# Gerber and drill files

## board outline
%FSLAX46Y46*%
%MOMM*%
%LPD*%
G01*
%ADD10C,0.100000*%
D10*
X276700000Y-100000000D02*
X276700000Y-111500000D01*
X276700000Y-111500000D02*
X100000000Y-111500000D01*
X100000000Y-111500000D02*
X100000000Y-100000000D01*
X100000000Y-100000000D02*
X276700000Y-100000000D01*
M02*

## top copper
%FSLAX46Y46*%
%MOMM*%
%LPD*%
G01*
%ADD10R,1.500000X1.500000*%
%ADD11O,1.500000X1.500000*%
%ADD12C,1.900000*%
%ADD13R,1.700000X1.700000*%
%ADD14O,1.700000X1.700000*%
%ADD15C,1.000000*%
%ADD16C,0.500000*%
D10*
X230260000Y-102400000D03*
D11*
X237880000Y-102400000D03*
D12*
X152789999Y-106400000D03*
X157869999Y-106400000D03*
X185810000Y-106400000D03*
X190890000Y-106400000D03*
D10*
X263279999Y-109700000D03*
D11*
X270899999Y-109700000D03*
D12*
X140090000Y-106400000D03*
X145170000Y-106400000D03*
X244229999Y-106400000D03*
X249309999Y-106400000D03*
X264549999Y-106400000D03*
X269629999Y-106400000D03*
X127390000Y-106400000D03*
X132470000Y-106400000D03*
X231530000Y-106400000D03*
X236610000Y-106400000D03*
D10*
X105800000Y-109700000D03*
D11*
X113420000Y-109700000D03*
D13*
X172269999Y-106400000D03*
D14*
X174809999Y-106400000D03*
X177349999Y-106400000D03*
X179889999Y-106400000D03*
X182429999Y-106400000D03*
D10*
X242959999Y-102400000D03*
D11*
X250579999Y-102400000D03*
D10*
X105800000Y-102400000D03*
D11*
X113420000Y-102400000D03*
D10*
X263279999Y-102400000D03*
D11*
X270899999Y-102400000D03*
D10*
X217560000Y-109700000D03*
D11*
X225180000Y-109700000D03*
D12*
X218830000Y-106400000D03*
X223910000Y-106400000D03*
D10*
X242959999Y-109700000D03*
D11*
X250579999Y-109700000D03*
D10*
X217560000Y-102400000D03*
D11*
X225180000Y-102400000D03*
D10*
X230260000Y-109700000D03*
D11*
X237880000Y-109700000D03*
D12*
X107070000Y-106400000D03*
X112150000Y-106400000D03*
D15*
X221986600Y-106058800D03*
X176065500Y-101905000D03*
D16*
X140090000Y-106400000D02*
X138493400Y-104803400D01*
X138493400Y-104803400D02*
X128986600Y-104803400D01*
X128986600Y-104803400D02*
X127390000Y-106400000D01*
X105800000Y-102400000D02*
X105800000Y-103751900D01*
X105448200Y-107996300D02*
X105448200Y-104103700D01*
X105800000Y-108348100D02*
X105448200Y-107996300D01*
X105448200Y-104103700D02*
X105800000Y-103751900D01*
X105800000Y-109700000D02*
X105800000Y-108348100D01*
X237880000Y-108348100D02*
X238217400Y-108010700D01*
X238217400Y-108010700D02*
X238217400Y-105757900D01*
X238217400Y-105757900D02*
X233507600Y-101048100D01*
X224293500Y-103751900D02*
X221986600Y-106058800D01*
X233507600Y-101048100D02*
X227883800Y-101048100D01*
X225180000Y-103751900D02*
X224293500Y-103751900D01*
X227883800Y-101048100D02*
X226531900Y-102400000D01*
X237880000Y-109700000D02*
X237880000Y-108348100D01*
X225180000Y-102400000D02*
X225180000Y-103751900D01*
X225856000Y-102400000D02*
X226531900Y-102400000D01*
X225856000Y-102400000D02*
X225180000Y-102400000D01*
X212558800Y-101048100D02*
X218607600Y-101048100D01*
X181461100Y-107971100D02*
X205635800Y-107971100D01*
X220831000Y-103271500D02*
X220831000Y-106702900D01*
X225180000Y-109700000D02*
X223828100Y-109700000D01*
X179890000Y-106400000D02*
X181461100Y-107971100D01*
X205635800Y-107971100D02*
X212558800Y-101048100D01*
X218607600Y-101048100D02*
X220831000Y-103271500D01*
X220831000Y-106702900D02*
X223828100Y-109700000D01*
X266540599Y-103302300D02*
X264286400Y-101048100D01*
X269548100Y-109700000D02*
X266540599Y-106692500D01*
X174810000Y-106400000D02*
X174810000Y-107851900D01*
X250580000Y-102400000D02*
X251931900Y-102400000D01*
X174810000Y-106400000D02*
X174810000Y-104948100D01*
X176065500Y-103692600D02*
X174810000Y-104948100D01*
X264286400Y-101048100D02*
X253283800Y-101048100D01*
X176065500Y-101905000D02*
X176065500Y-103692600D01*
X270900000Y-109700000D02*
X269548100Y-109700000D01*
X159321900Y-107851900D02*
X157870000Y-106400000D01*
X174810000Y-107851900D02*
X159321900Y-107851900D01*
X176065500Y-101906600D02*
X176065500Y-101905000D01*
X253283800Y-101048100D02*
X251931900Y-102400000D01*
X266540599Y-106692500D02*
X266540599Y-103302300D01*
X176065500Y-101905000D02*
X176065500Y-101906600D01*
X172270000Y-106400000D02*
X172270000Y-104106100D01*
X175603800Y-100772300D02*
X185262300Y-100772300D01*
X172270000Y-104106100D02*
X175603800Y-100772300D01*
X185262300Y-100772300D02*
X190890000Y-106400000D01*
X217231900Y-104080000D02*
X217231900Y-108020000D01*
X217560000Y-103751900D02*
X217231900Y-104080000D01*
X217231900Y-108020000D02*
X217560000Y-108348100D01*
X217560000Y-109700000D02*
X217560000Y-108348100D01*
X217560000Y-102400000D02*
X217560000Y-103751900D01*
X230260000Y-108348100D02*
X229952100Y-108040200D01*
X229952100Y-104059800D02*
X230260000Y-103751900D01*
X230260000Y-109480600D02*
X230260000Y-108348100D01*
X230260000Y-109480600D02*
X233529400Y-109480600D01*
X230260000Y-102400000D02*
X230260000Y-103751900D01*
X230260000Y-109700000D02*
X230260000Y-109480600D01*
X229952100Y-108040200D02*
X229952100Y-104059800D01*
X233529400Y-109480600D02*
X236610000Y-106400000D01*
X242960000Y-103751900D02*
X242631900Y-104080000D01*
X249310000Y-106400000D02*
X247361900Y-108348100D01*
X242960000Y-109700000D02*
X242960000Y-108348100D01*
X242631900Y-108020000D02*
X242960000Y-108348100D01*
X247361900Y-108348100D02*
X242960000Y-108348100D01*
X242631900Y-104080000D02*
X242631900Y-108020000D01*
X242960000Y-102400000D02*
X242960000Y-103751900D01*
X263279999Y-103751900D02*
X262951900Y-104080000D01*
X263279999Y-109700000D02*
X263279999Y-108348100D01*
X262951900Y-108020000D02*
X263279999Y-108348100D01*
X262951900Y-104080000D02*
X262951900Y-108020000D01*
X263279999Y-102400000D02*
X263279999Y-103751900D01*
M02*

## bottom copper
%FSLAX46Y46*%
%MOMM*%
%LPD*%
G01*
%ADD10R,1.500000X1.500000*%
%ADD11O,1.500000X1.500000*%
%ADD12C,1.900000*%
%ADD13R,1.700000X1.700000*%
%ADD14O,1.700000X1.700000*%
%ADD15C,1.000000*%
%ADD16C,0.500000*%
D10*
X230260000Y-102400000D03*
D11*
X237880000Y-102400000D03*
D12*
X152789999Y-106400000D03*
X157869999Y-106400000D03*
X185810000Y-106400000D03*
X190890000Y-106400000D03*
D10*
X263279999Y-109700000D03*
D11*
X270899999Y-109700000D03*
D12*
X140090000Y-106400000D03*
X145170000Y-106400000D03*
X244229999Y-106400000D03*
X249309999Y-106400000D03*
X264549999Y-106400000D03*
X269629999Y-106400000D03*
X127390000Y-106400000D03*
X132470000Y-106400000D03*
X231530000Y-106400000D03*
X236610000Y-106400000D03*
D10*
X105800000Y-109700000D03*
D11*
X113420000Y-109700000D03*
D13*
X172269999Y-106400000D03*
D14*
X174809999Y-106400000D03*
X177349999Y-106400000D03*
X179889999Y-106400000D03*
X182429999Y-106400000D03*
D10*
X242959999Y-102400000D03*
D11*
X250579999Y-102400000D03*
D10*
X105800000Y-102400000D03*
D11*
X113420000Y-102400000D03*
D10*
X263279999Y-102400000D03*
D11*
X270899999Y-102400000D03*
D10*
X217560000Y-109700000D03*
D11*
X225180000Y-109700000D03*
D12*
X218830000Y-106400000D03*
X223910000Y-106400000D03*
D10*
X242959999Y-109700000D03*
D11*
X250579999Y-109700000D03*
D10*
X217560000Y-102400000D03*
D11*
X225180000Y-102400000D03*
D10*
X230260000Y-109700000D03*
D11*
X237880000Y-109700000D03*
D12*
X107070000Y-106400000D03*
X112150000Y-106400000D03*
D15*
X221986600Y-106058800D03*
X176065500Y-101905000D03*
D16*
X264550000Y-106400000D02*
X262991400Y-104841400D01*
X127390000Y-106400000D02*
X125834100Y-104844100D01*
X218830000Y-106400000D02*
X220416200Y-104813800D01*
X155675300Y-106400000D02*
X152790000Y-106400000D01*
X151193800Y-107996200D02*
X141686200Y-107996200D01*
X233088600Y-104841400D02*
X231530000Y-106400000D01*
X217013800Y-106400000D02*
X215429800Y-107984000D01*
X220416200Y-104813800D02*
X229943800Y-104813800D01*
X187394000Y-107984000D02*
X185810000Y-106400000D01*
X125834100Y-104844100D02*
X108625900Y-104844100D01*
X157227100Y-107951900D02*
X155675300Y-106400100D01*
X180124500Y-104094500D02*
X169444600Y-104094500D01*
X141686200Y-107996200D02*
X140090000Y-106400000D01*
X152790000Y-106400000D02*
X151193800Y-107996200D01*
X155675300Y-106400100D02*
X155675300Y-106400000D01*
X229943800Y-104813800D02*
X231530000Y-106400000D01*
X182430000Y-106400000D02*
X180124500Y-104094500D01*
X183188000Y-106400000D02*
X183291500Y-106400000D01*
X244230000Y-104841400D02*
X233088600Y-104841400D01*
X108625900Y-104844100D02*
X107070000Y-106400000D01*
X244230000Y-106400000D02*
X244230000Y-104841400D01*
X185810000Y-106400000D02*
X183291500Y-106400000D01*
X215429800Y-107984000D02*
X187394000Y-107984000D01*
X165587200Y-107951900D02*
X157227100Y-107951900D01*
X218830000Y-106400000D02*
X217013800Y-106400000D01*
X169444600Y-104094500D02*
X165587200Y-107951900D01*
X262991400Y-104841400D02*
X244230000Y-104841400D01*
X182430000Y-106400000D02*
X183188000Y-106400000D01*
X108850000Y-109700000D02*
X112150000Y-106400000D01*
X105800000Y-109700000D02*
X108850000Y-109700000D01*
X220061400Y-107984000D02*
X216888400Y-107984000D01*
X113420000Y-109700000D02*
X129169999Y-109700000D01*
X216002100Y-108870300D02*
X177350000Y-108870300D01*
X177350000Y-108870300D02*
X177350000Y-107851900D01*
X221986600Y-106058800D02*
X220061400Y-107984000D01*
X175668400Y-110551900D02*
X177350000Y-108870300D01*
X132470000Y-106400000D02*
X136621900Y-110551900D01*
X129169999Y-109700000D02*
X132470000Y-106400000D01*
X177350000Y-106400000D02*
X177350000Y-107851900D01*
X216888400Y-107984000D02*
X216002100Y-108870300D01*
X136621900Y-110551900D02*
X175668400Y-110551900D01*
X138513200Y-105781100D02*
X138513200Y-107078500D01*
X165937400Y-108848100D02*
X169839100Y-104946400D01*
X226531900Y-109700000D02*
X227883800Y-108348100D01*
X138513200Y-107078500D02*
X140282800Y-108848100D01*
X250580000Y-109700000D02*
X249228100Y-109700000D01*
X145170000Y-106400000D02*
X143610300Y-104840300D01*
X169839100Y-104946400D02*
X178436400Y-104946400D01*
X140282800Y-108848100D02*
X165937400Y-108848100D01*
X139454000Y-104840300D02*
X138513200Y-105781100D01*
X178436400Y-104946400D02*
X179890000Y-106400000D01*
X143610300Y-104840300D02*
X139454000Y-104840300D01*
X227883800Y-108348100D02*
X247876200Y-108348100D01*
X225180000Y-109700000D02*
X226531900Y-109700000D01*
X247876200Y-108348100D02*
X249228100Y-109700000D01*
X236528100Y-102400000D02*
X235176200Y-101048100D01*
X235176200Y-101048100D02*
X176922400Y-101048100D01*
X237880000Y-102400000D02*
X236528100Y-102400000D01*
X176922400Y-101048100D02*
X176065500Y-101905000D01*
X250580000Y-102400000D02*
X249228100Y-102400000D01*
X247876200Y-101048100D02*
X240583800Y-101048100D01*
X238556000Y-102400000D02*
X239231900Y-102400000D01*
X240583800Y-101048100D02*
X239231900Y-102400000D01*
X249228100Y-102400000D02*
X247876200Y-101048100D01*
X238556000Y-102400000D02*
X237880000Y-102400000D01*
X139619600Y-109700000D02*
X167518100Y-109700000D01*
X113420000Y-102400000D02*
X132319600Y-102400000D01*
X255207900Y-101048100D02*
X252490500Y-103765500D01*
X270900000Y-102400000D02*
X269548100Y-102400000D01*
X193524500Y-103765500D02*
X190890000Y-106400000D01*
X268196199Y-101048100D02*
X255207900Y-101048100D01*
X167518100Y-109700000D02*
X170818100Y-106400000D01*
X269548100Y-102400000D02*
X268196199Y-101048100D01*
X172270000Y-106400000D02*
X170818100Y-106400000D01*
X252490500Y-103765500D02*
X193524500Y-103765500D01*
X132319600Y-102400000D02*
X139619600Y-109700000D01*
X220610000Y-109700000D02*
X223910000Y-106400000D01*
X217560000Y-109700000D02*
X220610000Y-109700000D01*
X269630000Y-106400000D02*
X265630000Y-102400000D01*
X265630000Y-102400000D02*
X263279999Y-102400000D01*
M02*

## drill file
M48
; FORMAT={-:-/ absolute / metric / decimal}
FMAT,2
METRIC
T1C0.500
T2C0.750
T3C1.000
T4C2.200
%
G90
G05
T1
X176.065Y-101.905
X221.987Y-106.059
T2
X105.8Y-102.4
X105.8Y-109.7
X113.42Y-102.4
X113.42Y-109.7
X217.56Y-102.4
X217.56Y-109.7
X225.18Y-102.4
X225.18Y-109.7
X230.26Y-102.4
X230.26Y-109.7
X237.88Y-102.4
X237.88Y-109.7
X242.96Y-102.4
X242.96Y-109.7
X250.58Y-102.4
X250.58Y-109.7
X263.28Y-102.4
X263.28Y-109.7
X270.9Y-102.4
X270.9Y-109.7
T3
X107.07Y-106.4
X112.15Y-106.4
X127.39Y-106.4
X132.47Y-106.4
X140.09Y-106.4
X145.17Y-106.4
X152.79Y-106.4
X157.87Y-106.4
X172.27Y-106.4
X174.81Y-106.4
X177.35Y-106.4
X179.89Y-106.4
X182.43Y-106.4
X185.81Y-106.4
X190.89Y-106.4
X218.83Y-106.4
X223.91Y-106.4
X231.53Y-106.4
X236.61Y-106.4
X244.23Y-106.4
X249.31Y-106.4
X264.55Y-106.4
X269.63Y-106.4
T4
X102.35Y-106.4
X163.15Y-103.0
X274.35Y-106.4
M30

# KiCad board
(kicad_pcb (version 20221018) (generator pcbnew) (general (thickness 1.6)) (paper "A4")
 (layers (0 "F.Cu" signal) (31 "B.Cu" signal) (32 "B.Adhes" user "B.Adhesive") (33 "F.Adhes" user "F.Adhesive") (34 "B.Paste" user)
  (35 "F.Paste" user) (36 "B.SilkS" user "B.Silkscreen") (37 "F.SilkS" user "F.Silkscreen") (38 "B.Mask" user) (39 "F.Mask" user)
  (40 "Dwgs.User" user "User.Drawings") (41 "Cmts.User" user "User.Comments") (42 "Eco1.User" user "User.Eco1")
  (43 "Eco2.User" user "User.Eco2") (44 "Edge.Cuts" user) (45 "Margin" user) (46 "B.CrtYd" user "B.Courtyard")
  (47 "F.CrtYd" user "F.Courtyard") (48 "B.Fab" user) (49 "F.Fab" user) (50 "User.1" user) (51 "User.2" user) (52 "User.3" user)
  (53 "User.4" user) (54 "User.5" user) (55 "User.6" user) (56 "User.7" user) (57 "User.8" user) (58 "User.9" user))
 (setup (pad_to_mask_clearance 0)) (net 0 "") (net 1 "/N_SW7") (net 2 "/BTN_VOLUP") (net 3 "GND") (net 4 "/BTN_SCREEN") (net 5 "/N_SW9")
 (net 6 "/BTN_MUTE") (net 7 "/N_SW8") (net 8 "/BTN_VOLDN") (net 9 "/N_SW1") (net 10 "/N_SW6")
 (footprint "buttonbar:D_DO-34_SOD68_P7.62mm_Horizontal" (layer "F.Cu") (at 230.26 102.4)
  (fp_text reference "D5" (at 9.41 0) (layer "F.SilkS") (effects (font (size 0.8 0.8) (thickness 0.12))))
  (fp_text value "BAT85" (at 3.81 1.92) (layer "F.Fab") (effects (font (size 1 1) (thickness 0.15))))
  (pad "1" thru_hole rect (at 0 0) (size 1.5 1.5) (drill 0.75) (layers "*.Cu" "*.Mask") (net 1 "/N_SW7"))
  (pad "2" thru_hole oval (at 7.62 0) (size 1.5 1.5) (drill 0.75) (layers "*.Cu" "*.Mask") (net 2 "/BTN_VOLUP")))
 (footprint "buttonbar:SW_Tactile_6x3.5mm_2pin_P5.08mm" (layer "F.Cu") (at 155.329999 106.4)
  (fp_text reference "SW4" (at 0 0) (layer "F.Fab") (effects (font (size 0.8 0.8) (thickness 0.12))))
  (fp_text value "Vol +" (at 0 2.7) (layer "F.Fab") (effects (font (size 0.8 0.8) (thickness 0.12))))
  (pad "1" thru_hole circle (at -2.54 0) (size 1.9 1.9) (drill 1) (layers "*.Cu" "*.Mask") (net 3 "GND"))
  (pad "2" thru_hole circle (at 2.54 0) (size 1.9 1.9) (drill 1) (layers "*.Cu" "*.Mask") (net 2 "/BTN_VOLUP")))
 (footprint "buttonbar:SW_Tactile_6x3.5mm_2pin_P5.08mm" (layer "F.Cu") (at 188.35 106.4)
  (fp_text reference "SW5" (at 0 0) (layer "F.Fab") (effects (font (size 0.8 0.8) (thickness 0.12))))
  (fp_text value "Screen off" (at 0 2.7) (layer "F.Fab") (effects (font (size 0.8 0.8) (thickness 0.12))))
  (pad "1" thru_hole circle (at -2.54 0) (size 1.9 1.9) (drill 1) (layers "*.Cu" "*.Mask") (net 3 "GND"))
  (pad "2" thru_hole circle (at 2.54 0) (size 1.9 1.9) (drill 1) (layers "*.Cu" "*.Mask") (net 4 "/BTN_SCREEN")))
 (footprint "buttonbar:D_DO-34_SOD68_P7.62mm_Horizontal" (layer "F.Cu") (at 263.279999 109.7)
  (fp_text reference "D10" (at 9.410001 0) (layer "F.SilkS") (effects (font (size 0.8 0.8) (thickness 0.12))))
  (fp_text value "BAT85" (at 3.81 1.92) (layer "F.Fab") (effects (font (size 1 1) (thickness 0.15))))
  (pad "1" thru_hole rect (at 0 0) (size 1.5 1.5) (drill 0.75) (layers "*.Cu" "*.Mask") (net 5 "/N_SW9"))
  (pad "2" thru_hole oval (at 7.62 0) (size 1.5 1.5) (drill 0.75) (layers "*.Cu" "*.Mask") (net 2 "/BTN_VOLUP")))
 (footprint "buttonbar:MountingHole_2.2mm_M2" (layer "F.Cu") (at 163.15 103)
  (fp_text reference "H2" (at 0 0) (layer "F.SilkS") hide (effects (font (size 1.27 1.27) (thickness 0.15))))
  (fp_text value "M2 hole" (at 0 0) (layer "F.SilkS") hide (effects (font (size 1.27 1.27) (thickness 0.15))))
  (pad "" np_thru_hole circle (at 0 0) (size 2.2 2.2) (drill 2.2) (layers "F&B.Cu" "*.Mask")))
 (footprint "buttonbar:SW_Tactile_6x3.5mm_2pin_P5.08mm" (layer "F.Cu") (at 142.63 106.4)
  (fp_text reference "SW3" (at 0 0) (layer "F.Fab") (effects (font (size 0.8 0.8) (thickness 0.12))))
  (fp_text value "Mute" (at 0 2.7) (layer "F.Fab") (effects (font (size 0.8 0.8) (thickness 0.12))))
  (pad "1" thru_hole circle (at -2.54 0) (size 1.9 1.9) (drill 1) (layers "*.Cu" "*.Mask") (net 3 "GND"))
  (pad "2" thru_hole circle (at 2.54 0) (size 1.9 1.9) (drill 1) (layers "*.Cu" "*.Mask") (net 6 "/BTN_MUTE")))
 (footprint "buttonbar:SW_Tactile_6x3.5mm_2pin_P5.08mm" (layer "F.Cu") (at 246.769999 106.4)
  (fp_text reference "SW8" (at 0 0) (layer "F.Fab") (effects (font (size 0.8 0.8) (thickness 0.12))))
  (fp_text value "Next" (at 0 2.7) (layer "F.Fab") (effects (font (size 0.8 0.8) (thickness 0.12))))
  (pad "1" thru_hole circle (at -2.54 0) (size 1.9 1.9) (drill 1) (layers "*.Cu" "*.Mask") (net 3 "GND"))
  (pad "2" thru_hole circle (at 2.54 0) (size 1.9 1.9) (drill 1) (layers "*.Cu" "*.Mask") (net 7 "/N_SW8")))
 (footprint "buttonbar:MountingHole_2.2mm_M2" (layer "F.Cu") (at 102.35 106.4)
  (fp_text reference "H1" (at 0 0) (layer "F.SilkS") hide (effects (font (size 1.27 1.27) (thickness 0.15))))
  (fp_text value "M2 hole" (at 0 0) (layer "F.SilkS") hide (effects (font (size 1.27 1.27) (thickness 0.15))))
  (pad "" np_thru_hole circle (at 0 0) (size 2.2 2.2) (drill 2.2) (layers "F&B.Cu" "*.Mask")))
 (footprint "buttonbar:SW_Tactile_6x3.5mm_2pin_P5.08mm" (layer "F.Cu") (at 267.089999 106.4)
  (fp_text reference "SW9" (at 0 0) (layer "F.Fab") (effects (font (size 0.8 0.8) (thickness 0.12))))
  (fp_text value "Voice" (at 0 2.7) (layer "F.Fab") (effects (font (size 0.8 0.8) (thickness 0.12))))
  (pad "1" thru_hole circle (at -2.54 0) (size 1.9 1.9) (drill 1) (layers "*.Cu" "*.Mask") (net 3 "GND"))
  (pad "2" thru_hole circle (at 2.54 0) (size 1.9 1.9) (drill 1) (layers "*.Cu" "*.Mask") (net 5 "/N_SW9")))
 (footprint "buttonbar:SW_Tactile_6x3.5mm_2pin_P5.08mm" (layer "F.Cu") (at 129.93 106.4)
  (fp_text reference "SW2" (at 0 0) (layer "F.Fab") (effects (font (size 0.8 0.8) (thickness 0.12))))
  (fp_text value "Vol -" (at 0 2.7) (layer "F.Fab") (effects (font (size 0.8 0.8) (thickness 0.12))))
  (pad "1" thru_hole circle (at -2.54 0) (size 1.9 1.9) (drill 1) (layers "*.Cu" "*.Mask") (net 3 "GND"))
  (pad "2" thru_hole circle (at 2.54 0) (size 1.9 1.9) (drill 1) (layers "*.Cu" "*.Mask") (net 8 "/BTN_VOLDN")))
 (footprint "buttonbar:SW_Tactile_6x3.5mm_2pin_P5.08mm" (layer "F.Cu") (at 234.07 106.4)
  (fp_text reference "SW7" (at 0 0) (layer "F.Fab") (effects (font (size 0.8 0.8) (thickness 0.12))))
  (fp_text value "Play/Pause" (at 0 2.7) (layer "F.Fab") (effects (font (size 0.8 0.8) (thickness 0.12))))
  (pad "1" thru_hole circle (at -2.54 0) (size 1.9 1.9) (drill 1) (layers "*.Cu" "*.Mask") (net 3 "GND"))
  (pad "2" thru_hole circle (at 2.54 0) (size 1.9 1.9) (drill 1) (layers "*.Cu" "*.Mask") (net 1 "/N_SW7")))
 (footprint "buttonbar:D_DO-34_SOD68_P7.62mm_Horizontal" (layer "F.Cu") (at 105.8 109.7)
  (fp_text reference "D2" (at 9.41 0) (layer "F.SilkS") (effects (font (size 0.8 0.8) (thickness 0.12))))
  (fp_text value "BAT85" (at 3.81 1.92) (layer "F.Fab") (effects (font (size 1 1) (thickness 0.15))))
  (pad "1" thru_hole rect (at 0 0) (size 1.5 1.5) (drill 0.75) (layers "*.Cu" "*.Mask") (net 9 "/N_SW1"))
  (pad "2" thru_hole oval (at 7.62 0) (size 1.5 1.5) (drill 0.75) (layers "*.Cu" "*.Mask") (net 8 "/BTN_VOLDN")))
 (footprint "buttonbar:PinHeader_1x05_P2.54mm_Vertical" (layer "F.Cu") (at 172.269999 106.4 90)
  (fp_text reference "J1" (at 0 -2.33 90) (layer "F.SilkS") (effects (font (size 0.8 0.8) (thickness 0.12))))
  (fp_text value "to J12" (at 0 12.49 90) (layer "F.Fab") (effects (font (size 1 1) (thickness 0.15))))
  (pad "1" thru_hole rect (at 0 0 90) (size 1.7 1.7) (drill 1) (layers "*.Cu" "*.Mask") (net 4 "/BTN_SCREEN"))
  (pad "2" thru_hole oval (at 0 2.54 90) (size 1.7 1.7) (drill 1) (layers "*.Cu" "*.Mask") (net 2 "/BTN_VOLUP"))
  (pad "3" thru_hole oval (at 0 5.08 90) (size 1.7 1.7) (drill 1) (layers "*.Cu" "*.Mask") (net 8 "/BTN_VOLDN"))
  (pad "4" thru_hole oval (at 0 7.62 90) (size 1.7 1.7) (drill 1) (layers "*.Cu" "*.Mask") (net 6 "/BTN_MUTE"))
  (pad "5" thru_hole oval (at 0 10.16 90) (size 1.7 1.7) (drill 1) (layers "*.Cu" "*.Mask") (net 3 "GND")))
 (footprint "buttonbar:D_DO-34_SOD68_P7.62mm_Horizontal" (layer "F.Cu") (at 242.959999 102.4)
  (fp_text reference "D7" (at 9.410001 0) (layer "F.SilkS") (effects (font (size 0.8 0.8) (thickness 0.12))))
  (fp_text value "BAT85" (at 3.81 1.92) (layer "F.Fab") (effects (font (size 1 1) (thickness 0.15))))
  (pad "1" thru_hole rect (at 0 0) (size 1.5 1.5) (drill 0.75) (layers "*.Cu" "*.Mask") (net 7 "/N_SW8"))
  (pad "2" thru_hole oval (at 7.62 0) (size 1.5 1.5) (drill 0.75) (layers "*.Cu" "*.Mask") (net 2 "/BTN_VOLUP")))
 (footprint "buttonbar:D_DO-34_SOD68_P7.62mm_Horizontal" (layer "F.Cu") (at 105.8 102.4)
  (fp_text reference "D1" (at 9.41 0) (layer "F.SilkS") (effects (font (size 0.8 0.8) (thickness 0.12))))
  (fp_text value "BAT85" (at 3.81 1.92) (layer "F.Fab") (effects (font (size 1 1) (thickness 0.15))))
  (pad "1" thru_hole rect (at 0 0) (size 1.5 1.5) (drill 0.75) (layers "*.Cu" "*.Mask") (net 9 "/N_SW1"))
  (pad "2" thru_hole oval (at 7.62 0) (size 1.5 1.5) (drill 0.75) (layers "*.Cu" "*.Mask") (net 4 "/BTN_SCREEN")))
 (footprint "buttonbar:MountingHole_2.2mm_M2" (layer "F.Cu") (at 274.35 106.4)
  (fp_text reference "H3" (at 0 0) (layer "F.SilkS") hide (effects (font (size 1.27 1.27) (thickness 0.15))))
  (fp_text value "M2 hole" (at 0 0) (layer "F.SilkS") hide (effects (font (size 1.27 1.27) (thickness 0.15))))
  (pad "" np_thru_hole circle (at 0 0) (size 2.2 2.2) (drill 2.2) (layers "F&B.Cu" "*.Mask")))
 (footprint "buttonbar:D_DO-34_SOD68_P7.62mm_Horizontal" (layer "F.Cu") (at 263.279999 102.4)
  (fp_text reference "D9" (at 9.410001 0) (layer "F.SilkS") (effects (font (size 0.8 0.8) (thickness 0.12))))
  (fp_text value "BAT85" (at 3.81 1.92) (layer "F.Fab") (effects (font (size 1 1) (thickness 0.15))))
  (pad "1" thru_hole rect (at 0 0) (size 1.5 1.5) (drill 0.75) (layers "*.Cu" "*.Mask") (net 5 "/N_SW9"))
  (pad "2" thru_hole oval (at 7.62 0) (size 1.5 1.5) (drill 0.75) (layers "*.Cu" "*.Mask") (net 4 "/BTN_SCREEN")))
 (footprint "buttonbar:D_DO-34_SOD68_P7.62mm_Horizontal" (layer "F.Cu") (at 217.56 109.7)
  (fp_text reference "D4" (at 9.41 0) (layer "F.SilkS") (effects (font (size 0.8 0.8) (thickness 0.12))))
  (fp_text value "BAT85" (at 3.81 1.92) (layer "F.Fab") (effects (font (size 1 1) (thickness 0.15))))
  (pad "1" thru_hole rect (at 0 0) (size 1.5 1.5) (drill 0.75) (layers "*.Cu" "*.Mask") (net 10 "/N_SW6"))
  (pad "2" thru_hole oval (at 7.62 0) (size 1.5 1.5) (drill 0.75) (layers "*.Cu" "*.Mask") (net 6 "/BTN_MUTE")))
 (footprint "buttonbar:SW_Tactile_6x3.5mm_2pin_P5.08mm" (layer "F.Cu") (at 221.37 106.4)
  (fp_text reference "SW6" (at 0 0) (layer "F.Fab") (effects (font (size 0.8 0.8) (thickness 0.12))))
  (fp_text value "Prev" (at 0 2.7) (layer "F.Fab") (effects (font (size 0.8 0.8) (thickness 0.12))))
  (pad "1" thru_hole circle (at -2.54 0) (size 1.9 1.9) (drill 1) (layers "*.Cu" "*.Mask") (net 3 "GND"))
  (pad "2" thru_hole circle (at 2.54 0) (size 1.9 1.9) (drill 1) (layers "*.Cu" "*.Mask") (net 10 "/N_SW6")))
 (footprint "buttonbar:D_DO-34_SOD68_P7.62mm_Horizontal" (layer "F.Cu") (at 242.959999 109.7)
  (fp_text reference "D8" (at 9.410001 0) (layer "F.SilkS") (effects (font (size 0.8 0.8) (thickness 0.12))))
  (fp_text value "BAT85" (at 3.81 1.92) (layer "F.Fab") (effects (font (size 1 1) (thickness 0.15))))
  (pad "1" thru_hole rect (at 0 0) (size 1.5 1.5) (drill 0.75) (layers "*.Cu" "*.Mask") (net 7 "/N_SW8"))
  (pad "2" thru_hole oval (at 7.62 0) (size 1.5 1.5) (drill 0.75) (layers "*.Cu" "*.Mask") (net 6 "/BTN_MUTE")))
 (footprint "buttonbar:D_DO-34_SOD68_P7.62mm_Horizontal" (layer "F.Cu") (at 217.56 102.4)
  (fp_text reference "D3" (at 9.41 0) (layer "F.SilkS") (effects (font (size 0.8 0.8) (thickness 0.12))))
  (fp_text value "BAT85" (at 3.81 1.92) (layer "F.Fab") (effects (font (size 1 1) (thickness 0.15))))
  (pad "1" thru_hole rect (at 0 0) (size 1.5 1.5) (drill 0.75) (layers "*.Cu" "*.Mask") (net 10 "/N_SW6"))
  (pad "2" thru_hole oval (at 7.62 0) (size 1.5 1.5) (drill 0.75) (layers "*.Cu" "*.Mask") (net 8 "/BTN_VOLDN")))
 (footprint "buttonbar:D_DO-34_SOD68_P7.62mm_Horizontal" (layer "F.Cu") (at 230.26 109.7)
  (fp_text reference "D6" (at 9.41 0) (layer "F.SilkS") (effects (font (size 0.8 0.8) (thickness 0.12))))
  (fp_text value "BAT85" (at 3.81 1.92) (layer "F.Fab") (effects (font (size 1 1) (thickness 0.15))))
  (pad "1" thru_hole rect (at 0 0) (size 1.5 1.5) (drill 0.75) (layers "*.Cu" "*.Mask") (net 1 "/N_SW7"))
  (pad "2" thru_hole oval (at 7.62 0) (size 1.5 1.5) (drill 0.75) (layers "*.Cu" "*.Mask") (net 8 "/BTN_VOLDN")))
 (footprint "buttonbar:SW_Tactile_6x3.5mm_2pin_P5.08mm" (layer "F.Cu") (at 109.61 106.4)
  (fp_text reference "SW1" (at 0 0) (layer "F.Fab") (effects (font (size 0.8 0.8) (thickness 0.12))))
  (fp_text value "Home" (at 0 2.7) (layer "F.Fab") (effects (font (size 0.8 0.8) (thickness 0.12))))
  (pad "1" thru_hole circle (at -2.54 0) (size 1.9 1.9) (drill 1) (layers "*.Cu" "*.Mask") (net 3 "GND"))
  (pad "2" thru_hole circle (at 2.54 0) (size 1.9 1.9) (drill 1) (layers "*.Cu" "*.Mask") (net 9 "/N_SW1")))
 (gr_line (start 276.7 100) (end 276.7 111.5) (stroke (width 0.1) (type default)) (layer "Edge.Cuts"))
 (gr_line (start 276.7 111.5) (end 100 111.5) (stroke (width 0.1) (type default)) (layer "Edge.Cuts"))
 (gr_line (start 100 111.5) (end 100 100) (stroke (width 0.1) (type default)) (layer "Edge.Cuts"))
 (gr_line (start 100 100) (end 276.7 100) (stroke (width 0.1) (type default)) (layer "Edge.Cuts"))
 (segment (start 140.09 106.4) (end 138.4934 104.8034) (width 0.5) (layer "F.Cu") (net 3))
 (segment (start 138.4934 104.8034) (end 128.9866 104.8034) (width 0.5) (layer "F.Cu") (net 3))
 (segment (start 128.9866 104.8034) (end 127.39 106.4) (width 0.5) (layer "F.Cu") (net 3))
 (segment (start 264.55 106.4) (end 262.9914 104.8414) (width 0.5) (layer "B.Cu") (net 3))
 (segment (start 127.39 106.4) (end 125.8341 104.8441) (width 0.5) (layer "B.Cu") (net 3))
 (segment (start 218.83 106.4) (end 220.4162 104.8138) (width 0.5) (layer "B.Cu") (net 3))
 (segment (start 155.6753 106.4) (end 152.79 106.4) (width 0.5) (layer "B.Cu") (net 3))
 (segment (start 151.1938 107.9962) (end 141.6862 107.9962) (width 0.5) (layer "B.Cu") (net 3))
 (segment (start 233.0886 104.8414) (end 231.53 106.4) (width 0.5) (layer "B.Cu") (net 3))
 (segment (start 217.0138 106.4) (end 215.4298 107.984) (width 0.5) (layer "B.Cu") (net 3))
 (segment (start 220.4162 104.8138) (end 229.9438 104.8138) (width 0.5) (layer "B.Cu") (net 3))
 (segment (start 187.394 107.984) (end 185.81 106.4) (width 0.5) (layer "B.Cu") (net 3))
 (segment (start 125.8341 104.8441) (end 108.6259 104.8441) (width 0.5) (layer "B.Cu") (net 3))
 (segment (start 157.2271 107.9519) (end 155.6753 106.4001) (width 0.5) (layer "B.Cu") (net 3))
 (segment (start 180.1245 104.0945) (end 169.4446 104.0945) (width 0.5) (layer "B.Cu") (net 3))
 (segment (start 141.6862 107.9962) (end 140.09 106.4) (width 0.5) (layer "B.Cu") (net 3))
 (segment (start 152.79 106.4) (end 151.1938 107.9962) (width 0.5) (layer "B.Cu") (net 3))
 (segment (start 155.6753 106.4001) (end 155.6753 106.4) (width 0.5) (layer "B.Cu") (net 3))
 (segment (start 229.9438 104.8138) (end 231.53 106.4) (width 0.5) (layer "B.Cu") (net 3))
 (segment (start 182.43 106.4) (end 180.1245 104.0945) (width 0.5) (layer "B.Cu") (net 3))
 (segment (start 183.188 106.4) (end 183.2915 106.4) (width 0.5) (layer "B.Cu") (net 3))
 (segment (start 244.23 104.8414) (end 233.0886 104.8414) (width 0.5) (layer "B.Cu") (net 3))
 (segment (start 108.6259 104.8441) (end 107.07 106.4) (width 0.5) (layer "B.Cu") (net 3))
 (segment (start 244.23 106.4) (end 244.23 104.8414) (width 0.5) (layer "B.Cu") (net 3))
 (segment (start 185.81 106.4) (end 183.2915 106.4) (width 0.5) (layer "B.Cu") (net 3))
 (segment (start 215.4298 107.984) (end 187.394 107.984) (width 0.5) (layer "B.Cu") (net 3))
 (segment (start 165.5872 107.9519) (end 157.2271 107.9519) (width 0.5) (layer "B.Cu") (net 3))
 (segment (start 218.83 106.4) (end 217.0138 106.4) (width 0.5) (layer "B.Cu") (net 3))
 (segment (start 169.4446 104.0945) (end 165.5872 107.9519) (width 0.5) (layer "B.Cu") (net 3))
 (segment (start 262.9914 104.8414) (end 244.23 104.8414) (width 0.5) (layer "B.Cu") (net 3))
 (segment (start 182.43 106.4) (end 183.188 106.4) (width 0.5) (layer "B.Cu") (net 3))
 (segment (start 105.8 102.4) (end 105.8 103.7519) (width 0.5) (layer "F.Cu") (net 9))
 (segment (start 105.4482 107.9963) (end 105.4482 104.1037) (width 0.5) (layer "F.Cu") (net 9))
 (segment (start 105.8 108.3481) (end 105.4482 107.9963) (width 0.5) (layer "F.Cu") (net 9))
 (segment (start 105.4482 104.1037) (end 105.8 103.7519) (width 0.5) (layer "F.Cu") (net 9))
 (segment (start 105.8 109.7) (end 105.8 108.3481) (width 0.5) (layer "F.Cu") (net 9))
 (segment (start 108.85 109.7) (end 112.15 106.4) (width 0.5) (layer "B.Cu") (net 9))
 (segment (start 105.8 109.7) (end 108.85 109.7) (width 0.5) (layer "B.Cu") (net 9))
 (segment (start 237.88 108.3481) (end 238.2174 108.0107) (width 0.5) (layer "F.Cu") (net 8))
 (segment (start 238.2174 108.0107) (end 238.2174 105.7579) (width 0.5) (layer "F.Cu") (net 8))
 (segment (start 238.2174 105.7579) (end 233.5076 101.0481) (width 0.5) (layer "F.Cu") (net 8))
 (segment (start 224.2935 103.7519) (end 221.9866 106.0588) (width 0.5) (layer "F.Cu") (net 8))
 (segment (start 233.5076 101.0481) (end 227.8838 101.0481) (width 0.5) (layer "F.Cu") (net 8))
 (segment (start 225.18 103.7519) (end 224.2935 103.7519) (width 0.5) (layer "F.Cu") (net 8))
 (segment (start 227.8838 101.0481) (end 226.5319 102.4) (width 0.5) (layer "F.Cu") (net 8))
 (segment (start 237.88 109.7) (end 237.88 108.3481) (width 0.5) (layer "F.Cu") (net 8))
 (segment (start 225.18 102.4) (end 225.18 103.7519) (width 0.5) (layer "F.Cu") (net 8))
 (segment (start 225.856 102.4) (end 226.5319 102.4) (width 0.5) (layer "F.Cu") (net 8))
 (segment (start 225.856 102.4) (end 225.18 102.4) (width 0.5) (layer "F.Cu") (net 8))
 (via (at 221.9866 106.0588) (size 1) (drill 0.5) (layers "F.Cu" "B.Cu") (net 8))
 (segment (start 220.0614 107.984) (end 216.8884 107.984) (width 0.5) (layer "B.Cu") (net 8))
 (segment (start 113.42 109.7) (end 129.169999 109.7) (width 0.5) (layer "B.Cu") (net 8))
 (segment (start 216.0021 108.8703) (end 177.35 108.8703) (width 0.5) (layer "B.Cu") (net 8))
 (segment (start 177.35 108.8703) (end 177.35 107.8519) (width 0.5) (layer "B.Cu") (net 8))
 (segment (start 221.9866 106.0588) (end 220.0614 107.984) (width 0.5) (layer "B.Cu") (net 8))
 (segment (start 175.6684 110.5519) (end 177.35 108.8703) (width 0.5) (layer "B.Cu") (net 8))
 (segment (start 132.47 106.4) (end 136.6219 110.5519) (width 0.5) (layer "B.Cu") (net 8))
 (segment (start 129.169999 109.7) (end 132.47 106.4) (width 0.5) (layer "B.Cu") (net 8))
 (segment (start 177.35 106.4) (end 177.35 107.8519) (width 0.5) (layer "B.Cu") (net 8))
 (segment (start 216.8884 107.984) (end 216.0021 108.8703) (width 0.5) (layer "B.Cu") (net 8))
 (segment (start 136.6219 110.5519) (end 175.6684 110.5519) (width 0.5) (layer "B.Cu") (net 8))
 (segment (start 212.5588 101.0481) (end 218.6076 101.0481) (width 0.5) (layer "F.Cu") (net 6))
 (segment (start 181.4611 107.9711) (end 205.6358 107.9711) (width 0.5) (layer "F.Cu") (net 6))
 (segment (start 220.831 103.2715) (end 220.831 106.7029) (width 0.5) (layer "F.Cu") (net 6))
 (segment (start 225.18 109.7) (end 223.8281 109.7) (width 0.5) (layer "F.Cu") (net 6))
 (segment (start 179.89 106.4) (end 181.4611 107.9711) (width 0.5) (layer "F.Cu") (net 6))
 (segment (start 205.6358 107.9711) (end 212.5588 101.0481) (width 0.5) (layer "F.Cu") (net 6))
 (segment (start 218.6076 101.0481) (end 220.831 103.2715) (width 0.5) (layer "F.Cu") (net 6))
 (segment (start 220.831 106.7029) (end 223.8281 109.7) (width 0.5) (layer "F.Cu") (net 6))
 (segment (start 138.5132 105.7811) (end 138.5132 107.0785) (width 0.5) (layer "B.Cu") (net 6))
 (segment (start 165.9374 108.8481) (end 169.8391 104.9464) (width 0.5) (layer "B.Cu") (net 6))
 (segment (start 226.5319 109.7) (end 227.8838 108.3481) (width 0.5) (layer "B.Cu") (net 6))
 (segment (start 138.5132 107.0785) (end 140.2828 108.8481) (width 0.5) (layer "B.Cu") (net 6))
 (segment (start 250.58 109.7) (end 249.2281 109.7) (width 0.5) (layer "B.Cu") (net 6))
 (segment (start 145.17 106.4) (end 143.6103 104.8403) (width 0.5) (layer "B.Cu") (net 6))
 (segment (start 169.8391 104.9464) (end 178.4364 104.9464) (width 0.5) (layer "B.Cu") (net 6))
 (segment (start 140.2828 108.8481) (end 165.9374 108.8481) (width 0.5) (layer "B.Cu") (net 6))
 (segment (start 139.454 104.8403) (end 138.5132 105.7811) (width 0.5) (layer "B.Cu") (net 6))
 (segment (start 178.4364 104.9464) (end 179.89 106.4) (width 0.5) (layer "B.Cu") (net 6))
 (segment (start 143.6103 104.8403) (end 139.454 104.8403) (width 0.5) (layer "B.Cu") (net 6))
 (segment (start 227.8838 108.3481) (end 247.8762 108.3481) (width 0.5) (layer "B.Cu") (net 6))
 (segment (start 225.18 109.7) (end 226.5319 109.7) (width 0.5) (layer "B.Cu") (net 6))
 (segment (start 247.8762 108.3481) (end 249.2281 109.7) (width 0.5) (layer "B.Cu") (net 6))
 (segment (start 266.540599 103.3023) (end 264.2864 101.0481) (width 0.5) (layer "F.Cu") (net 2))
 (segment (start 269.5481 109.7) (end 266.540599 106.6925) (width 0.5) (layer "F.Cu") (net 2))
 (segment (start 174.81 106.4) (end 174.81 107.8519) (width 0.5) (layer "F.Cu") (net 2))
 (segment (start 250.58 102.4) (end 251.9319 102.4) (width 0.5) (layer "F.Cu") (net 2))
 (segment (start 174.81 106.4) (end 174.81 104.9481) (width 0.5) (layer "F.Cu") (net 2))
 (segment (start 176.0655 103.6926) (end 174.81 104.9481) (width 0.5) (layer "F.Cu") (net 2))
 (segment (start 264.2864 101.0481) (end 253.2838 101.0481) (width 0.5) (layer "F.Cu") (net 2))
 (segment (start 176.0655 101.905) (end 176.0655 103.6926) (width 0.5) (layer "F.Cu") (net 2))
 (segment (start 270.9 109.7) (end 269.5481 109.7) (width 0.5) (layer "F.Cu") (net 2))
 (segment (start 159.3219 107.8519) (end 157.87 106.4) (width 0.5) (layer "F.Cu") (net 2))
 (segment (start 174.81 107.8519) (end 159.3219 107.8519) (width 0.5) (layer "F.Cu") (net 2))
 (segment (start 176.0655 101.9066) (end 176.0655 101.905) (width 0.5) (layer "F.Cu") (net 2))
 (segment (start 253.2838 101.0481) (end 251.9319 102.4) (width 0.5) (layer "F.Cu") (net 2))
 (segment (start 266.540599 106.6925) (end 266.540599 103.3023) (width 0.5) (layer "F.Cu") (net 2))
 (segment (start 176.0655 101.905) (end 176.0655 101.9066) (width 0.5) (layer "F.Cu") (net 2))
 (via (at 176.0655 101.905) (size 1) (drill 0.5) (layers "F.Cu" "B.Cu") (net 2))
 (segment (start 236.5281 102.4) (end 235.1762 101.0481) (width 0.5) (layer "B.Cu") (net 2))
 (segment (start 235.1762 101.0481) (end 176.9224 101.0481) (width 0.5) (layer "B.Cu") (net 2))
 (segment (start 237.88 102.4) (end 236.5281 102.4) (width 0.5) (layer "B.Cu") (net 2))
 (segment (start 176.9224 101.0481) (end 176.0655 101.905) (width 0.5) (layer "B.Cu") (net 2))
 (segment (start 250.58 102.4) (end 249.2281 102.4) (width 0.5) (layer "B.Cu") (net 2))
 (segment (start 247.8762 101.0481) (end 240.5838 101.0481) (width 0.5) (layer "B.Cu") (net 2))
 (segment (start 238.556 102.4) (end 239.2319 102.4) (width 0.5) (layer "B.Cu") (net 2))
 (segment (start 240.5838 101.0481) (end 239.2319 102.4) (width 0.5) (layer "B.Cu") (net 2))
 (segment (start 249.2281 102.4) (end 247.8762 101.0481) (width 0.5) (layer "B.Cu") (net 2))
 (segment (start 238.556 102.4) (end 237.88 102.4) (width 0.5) (layer "B.Cu") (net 2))
 (segment (start 172.27 106.4) (end 172.27 104.1061) (width 0.5) (layer "F.Cu") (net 4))
 (segment (start 175.6038 100.7723) (end 185.2623 100.7723) (width 0.5) (layer "F.Cu") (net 4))
 (segment (start 172.27 104.1061) (end 175.6038 100.7723) (width 0.5) (layer "F.Cu") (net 4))
 (segment (start 185.2623 100.7723) (end 190.89 106.4) (width 0.5) (layer "F.Cu") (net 4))
 (segment (start 139.6196 109.7) (end 167.5181 109.7) (width 0.5) (layer "B.Cu") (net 4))
 (segment (start 113.42 102.4) (end 132.3196 102.4) (width 0.5) (layer "B.Cu") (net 4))
 (segment (start 255.2079 101.0481) (end 252.4905 103.7655) (width 0.5) (layer "B.Cu") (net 4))
 (segment (start 270.9 102.4) (end 269.5481 102.4) (width 0.5) (layer "B.Cu") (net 4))
 (segment (start 193.5245 103.7655) (end 190.89 106.4) (width 0.5) (layer "B.Cu") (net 4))
 (segment (start 268.196199 101.0481) (end 255.2079 101.0481) (width 0.5) (layer "B.Cu") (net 4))
 (segment (start 167.5181 109.7) (end 170.8181 106.4) (width 0.5) (layer "B.Cu") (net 4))
 (segment (start 269.5481 102.4) (end 268.196199 101.0481) (width 0.5) (layer "B.Cu") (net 4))
 (segment (start 172.27 106.4) (end 170.8181 106.4) (width 0.5) (layer "B.Cu") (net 4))
 (segment (start 252.4905 103.7655) (end 193.5245 103.7655) (width 0.5) (layer "B.Cu") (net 4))
 (segment (start 132.3196 102.4) (end 139.6196 109.7) (width 0.5) (layer "B.Cu") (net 4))
 (segment (start 217.2319 104.08) (end 217.2319 108.02) (width 0.5) (layer "F.Cu") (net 10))
 (segment (start 217.56 103.7519) (end 217.2319 104.08) (width 0.5) (layer "F.Cu") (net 10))
 (segment (start 217.2319 108.02) (end 217.56 108.3481) (width 0.5) (layer "F.Cu") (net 10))
 (segment (start 217.56 109.7) (end 217.56 108.3481) (width 0.5) (layer "F.Cu") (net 10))
 (segment (start 217.56 102.4) (end 217.56 103.7519) (width 0.5) (layer "F.Cu") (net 10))
 (segment (start 220.61 109.7) (end 223.91 106.4) (width 0.5) (layer "B.Cu") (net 10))
 (segment (start 217.56 109.7) (end 220.61 109.7) (width 0.5) (layer "B.Cu") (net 10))
 (segment (start 230.26 108.3481) (end 229.9521 108.0402) (width 0.5) (layer "F.Cu") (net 1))
 (segment (start 229.9521 104.0598) (end 230.26 103.7519) (width 0.5) (layer "F.Cu") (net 1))
 (segment (start 230.26 109.4806) (end 230.26 108.3481) (width 0.5) (layer "F.Cu") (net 1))
 (segment (start 230.26 109.4806) (end 233.5294 109.4806) (width 0.5) (layer "F.Cu") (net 1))
 (segment (start 230.26 102.4) (end 230.26 103.7519) (width 0.5) (layer "F.Cu") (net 1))
 (segment (start 230.26 109.7) (end 230.26 109.4806) (width 0.5) (layer "F.Cu") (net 1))
 (segment (start 229.9521 108.0402) (end 229.9521 104.0598) (width 0.5) (layer "F.Cu") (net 1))
 (segment (start 233.5294 109.4806) (end 236.61 106.4) (width 0.5) (layer "F.Cu") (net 1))
 (segment (start 242.96 103.7519) (end 242.6319 104.08) (width 0.5) (layer "F.Cu") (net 7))
 (segment (start 249.31 106.4) (end 247.3619 108.3481) (width 0.5) (layer "F.Cu") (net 7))
 (segment (start 242.96 109.7) (end 242.96 108.3481) (width 0.5) (layer "F.Cu") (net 7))
 (segment (start 242.6319 108.02) (end 242.96 108.3481) (width 0.5) (layer "F.Cu") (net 7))
 (segment (start 247.3619 108.3481) (end 242.96 108.3481) (width 0.5) (layer "F.Cu") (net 7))
 (segment (start 242.6319 104.08) (end 242.6319 108.02) (width 0.5) (layer "F.Cu") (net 7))
 (segment (start 242.96 102.4) (end 242.96 103.7519) (width 0.5) (layer "F.Cu") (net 7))
 (segment (start 263.279999 103.7519) (end 262.9519 104.08) (width 0.5) (layer "F.Cu") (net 5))
 (segment (start 263.279999 109.7) (end 263.279999 108.3481) (width 0.5) (layer "F.Cu") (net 5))
 (segment (start 262.9519 108.02) (end 263.279999 108.3481) (width 0.5) (layer "F.Cu") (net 5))
 (segment (start 262.9519 104.08) (end 262.9519 108.02) (width 0.5) (layer "F.Cu") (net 5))
 (segment (start 263.279999 102.4) (end 263.279999 103.7519) (width 0.5) (layer "F.Cu") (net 5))
 (segment (start 269.63 106.4) (end 265.63 102.4) (width 0.5) (layer "B.Cu") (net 5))
 (segment (start 265.63 102.4) (end 263.279999 102.4) (width 0.5) (layer "B.Cu") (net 5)))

